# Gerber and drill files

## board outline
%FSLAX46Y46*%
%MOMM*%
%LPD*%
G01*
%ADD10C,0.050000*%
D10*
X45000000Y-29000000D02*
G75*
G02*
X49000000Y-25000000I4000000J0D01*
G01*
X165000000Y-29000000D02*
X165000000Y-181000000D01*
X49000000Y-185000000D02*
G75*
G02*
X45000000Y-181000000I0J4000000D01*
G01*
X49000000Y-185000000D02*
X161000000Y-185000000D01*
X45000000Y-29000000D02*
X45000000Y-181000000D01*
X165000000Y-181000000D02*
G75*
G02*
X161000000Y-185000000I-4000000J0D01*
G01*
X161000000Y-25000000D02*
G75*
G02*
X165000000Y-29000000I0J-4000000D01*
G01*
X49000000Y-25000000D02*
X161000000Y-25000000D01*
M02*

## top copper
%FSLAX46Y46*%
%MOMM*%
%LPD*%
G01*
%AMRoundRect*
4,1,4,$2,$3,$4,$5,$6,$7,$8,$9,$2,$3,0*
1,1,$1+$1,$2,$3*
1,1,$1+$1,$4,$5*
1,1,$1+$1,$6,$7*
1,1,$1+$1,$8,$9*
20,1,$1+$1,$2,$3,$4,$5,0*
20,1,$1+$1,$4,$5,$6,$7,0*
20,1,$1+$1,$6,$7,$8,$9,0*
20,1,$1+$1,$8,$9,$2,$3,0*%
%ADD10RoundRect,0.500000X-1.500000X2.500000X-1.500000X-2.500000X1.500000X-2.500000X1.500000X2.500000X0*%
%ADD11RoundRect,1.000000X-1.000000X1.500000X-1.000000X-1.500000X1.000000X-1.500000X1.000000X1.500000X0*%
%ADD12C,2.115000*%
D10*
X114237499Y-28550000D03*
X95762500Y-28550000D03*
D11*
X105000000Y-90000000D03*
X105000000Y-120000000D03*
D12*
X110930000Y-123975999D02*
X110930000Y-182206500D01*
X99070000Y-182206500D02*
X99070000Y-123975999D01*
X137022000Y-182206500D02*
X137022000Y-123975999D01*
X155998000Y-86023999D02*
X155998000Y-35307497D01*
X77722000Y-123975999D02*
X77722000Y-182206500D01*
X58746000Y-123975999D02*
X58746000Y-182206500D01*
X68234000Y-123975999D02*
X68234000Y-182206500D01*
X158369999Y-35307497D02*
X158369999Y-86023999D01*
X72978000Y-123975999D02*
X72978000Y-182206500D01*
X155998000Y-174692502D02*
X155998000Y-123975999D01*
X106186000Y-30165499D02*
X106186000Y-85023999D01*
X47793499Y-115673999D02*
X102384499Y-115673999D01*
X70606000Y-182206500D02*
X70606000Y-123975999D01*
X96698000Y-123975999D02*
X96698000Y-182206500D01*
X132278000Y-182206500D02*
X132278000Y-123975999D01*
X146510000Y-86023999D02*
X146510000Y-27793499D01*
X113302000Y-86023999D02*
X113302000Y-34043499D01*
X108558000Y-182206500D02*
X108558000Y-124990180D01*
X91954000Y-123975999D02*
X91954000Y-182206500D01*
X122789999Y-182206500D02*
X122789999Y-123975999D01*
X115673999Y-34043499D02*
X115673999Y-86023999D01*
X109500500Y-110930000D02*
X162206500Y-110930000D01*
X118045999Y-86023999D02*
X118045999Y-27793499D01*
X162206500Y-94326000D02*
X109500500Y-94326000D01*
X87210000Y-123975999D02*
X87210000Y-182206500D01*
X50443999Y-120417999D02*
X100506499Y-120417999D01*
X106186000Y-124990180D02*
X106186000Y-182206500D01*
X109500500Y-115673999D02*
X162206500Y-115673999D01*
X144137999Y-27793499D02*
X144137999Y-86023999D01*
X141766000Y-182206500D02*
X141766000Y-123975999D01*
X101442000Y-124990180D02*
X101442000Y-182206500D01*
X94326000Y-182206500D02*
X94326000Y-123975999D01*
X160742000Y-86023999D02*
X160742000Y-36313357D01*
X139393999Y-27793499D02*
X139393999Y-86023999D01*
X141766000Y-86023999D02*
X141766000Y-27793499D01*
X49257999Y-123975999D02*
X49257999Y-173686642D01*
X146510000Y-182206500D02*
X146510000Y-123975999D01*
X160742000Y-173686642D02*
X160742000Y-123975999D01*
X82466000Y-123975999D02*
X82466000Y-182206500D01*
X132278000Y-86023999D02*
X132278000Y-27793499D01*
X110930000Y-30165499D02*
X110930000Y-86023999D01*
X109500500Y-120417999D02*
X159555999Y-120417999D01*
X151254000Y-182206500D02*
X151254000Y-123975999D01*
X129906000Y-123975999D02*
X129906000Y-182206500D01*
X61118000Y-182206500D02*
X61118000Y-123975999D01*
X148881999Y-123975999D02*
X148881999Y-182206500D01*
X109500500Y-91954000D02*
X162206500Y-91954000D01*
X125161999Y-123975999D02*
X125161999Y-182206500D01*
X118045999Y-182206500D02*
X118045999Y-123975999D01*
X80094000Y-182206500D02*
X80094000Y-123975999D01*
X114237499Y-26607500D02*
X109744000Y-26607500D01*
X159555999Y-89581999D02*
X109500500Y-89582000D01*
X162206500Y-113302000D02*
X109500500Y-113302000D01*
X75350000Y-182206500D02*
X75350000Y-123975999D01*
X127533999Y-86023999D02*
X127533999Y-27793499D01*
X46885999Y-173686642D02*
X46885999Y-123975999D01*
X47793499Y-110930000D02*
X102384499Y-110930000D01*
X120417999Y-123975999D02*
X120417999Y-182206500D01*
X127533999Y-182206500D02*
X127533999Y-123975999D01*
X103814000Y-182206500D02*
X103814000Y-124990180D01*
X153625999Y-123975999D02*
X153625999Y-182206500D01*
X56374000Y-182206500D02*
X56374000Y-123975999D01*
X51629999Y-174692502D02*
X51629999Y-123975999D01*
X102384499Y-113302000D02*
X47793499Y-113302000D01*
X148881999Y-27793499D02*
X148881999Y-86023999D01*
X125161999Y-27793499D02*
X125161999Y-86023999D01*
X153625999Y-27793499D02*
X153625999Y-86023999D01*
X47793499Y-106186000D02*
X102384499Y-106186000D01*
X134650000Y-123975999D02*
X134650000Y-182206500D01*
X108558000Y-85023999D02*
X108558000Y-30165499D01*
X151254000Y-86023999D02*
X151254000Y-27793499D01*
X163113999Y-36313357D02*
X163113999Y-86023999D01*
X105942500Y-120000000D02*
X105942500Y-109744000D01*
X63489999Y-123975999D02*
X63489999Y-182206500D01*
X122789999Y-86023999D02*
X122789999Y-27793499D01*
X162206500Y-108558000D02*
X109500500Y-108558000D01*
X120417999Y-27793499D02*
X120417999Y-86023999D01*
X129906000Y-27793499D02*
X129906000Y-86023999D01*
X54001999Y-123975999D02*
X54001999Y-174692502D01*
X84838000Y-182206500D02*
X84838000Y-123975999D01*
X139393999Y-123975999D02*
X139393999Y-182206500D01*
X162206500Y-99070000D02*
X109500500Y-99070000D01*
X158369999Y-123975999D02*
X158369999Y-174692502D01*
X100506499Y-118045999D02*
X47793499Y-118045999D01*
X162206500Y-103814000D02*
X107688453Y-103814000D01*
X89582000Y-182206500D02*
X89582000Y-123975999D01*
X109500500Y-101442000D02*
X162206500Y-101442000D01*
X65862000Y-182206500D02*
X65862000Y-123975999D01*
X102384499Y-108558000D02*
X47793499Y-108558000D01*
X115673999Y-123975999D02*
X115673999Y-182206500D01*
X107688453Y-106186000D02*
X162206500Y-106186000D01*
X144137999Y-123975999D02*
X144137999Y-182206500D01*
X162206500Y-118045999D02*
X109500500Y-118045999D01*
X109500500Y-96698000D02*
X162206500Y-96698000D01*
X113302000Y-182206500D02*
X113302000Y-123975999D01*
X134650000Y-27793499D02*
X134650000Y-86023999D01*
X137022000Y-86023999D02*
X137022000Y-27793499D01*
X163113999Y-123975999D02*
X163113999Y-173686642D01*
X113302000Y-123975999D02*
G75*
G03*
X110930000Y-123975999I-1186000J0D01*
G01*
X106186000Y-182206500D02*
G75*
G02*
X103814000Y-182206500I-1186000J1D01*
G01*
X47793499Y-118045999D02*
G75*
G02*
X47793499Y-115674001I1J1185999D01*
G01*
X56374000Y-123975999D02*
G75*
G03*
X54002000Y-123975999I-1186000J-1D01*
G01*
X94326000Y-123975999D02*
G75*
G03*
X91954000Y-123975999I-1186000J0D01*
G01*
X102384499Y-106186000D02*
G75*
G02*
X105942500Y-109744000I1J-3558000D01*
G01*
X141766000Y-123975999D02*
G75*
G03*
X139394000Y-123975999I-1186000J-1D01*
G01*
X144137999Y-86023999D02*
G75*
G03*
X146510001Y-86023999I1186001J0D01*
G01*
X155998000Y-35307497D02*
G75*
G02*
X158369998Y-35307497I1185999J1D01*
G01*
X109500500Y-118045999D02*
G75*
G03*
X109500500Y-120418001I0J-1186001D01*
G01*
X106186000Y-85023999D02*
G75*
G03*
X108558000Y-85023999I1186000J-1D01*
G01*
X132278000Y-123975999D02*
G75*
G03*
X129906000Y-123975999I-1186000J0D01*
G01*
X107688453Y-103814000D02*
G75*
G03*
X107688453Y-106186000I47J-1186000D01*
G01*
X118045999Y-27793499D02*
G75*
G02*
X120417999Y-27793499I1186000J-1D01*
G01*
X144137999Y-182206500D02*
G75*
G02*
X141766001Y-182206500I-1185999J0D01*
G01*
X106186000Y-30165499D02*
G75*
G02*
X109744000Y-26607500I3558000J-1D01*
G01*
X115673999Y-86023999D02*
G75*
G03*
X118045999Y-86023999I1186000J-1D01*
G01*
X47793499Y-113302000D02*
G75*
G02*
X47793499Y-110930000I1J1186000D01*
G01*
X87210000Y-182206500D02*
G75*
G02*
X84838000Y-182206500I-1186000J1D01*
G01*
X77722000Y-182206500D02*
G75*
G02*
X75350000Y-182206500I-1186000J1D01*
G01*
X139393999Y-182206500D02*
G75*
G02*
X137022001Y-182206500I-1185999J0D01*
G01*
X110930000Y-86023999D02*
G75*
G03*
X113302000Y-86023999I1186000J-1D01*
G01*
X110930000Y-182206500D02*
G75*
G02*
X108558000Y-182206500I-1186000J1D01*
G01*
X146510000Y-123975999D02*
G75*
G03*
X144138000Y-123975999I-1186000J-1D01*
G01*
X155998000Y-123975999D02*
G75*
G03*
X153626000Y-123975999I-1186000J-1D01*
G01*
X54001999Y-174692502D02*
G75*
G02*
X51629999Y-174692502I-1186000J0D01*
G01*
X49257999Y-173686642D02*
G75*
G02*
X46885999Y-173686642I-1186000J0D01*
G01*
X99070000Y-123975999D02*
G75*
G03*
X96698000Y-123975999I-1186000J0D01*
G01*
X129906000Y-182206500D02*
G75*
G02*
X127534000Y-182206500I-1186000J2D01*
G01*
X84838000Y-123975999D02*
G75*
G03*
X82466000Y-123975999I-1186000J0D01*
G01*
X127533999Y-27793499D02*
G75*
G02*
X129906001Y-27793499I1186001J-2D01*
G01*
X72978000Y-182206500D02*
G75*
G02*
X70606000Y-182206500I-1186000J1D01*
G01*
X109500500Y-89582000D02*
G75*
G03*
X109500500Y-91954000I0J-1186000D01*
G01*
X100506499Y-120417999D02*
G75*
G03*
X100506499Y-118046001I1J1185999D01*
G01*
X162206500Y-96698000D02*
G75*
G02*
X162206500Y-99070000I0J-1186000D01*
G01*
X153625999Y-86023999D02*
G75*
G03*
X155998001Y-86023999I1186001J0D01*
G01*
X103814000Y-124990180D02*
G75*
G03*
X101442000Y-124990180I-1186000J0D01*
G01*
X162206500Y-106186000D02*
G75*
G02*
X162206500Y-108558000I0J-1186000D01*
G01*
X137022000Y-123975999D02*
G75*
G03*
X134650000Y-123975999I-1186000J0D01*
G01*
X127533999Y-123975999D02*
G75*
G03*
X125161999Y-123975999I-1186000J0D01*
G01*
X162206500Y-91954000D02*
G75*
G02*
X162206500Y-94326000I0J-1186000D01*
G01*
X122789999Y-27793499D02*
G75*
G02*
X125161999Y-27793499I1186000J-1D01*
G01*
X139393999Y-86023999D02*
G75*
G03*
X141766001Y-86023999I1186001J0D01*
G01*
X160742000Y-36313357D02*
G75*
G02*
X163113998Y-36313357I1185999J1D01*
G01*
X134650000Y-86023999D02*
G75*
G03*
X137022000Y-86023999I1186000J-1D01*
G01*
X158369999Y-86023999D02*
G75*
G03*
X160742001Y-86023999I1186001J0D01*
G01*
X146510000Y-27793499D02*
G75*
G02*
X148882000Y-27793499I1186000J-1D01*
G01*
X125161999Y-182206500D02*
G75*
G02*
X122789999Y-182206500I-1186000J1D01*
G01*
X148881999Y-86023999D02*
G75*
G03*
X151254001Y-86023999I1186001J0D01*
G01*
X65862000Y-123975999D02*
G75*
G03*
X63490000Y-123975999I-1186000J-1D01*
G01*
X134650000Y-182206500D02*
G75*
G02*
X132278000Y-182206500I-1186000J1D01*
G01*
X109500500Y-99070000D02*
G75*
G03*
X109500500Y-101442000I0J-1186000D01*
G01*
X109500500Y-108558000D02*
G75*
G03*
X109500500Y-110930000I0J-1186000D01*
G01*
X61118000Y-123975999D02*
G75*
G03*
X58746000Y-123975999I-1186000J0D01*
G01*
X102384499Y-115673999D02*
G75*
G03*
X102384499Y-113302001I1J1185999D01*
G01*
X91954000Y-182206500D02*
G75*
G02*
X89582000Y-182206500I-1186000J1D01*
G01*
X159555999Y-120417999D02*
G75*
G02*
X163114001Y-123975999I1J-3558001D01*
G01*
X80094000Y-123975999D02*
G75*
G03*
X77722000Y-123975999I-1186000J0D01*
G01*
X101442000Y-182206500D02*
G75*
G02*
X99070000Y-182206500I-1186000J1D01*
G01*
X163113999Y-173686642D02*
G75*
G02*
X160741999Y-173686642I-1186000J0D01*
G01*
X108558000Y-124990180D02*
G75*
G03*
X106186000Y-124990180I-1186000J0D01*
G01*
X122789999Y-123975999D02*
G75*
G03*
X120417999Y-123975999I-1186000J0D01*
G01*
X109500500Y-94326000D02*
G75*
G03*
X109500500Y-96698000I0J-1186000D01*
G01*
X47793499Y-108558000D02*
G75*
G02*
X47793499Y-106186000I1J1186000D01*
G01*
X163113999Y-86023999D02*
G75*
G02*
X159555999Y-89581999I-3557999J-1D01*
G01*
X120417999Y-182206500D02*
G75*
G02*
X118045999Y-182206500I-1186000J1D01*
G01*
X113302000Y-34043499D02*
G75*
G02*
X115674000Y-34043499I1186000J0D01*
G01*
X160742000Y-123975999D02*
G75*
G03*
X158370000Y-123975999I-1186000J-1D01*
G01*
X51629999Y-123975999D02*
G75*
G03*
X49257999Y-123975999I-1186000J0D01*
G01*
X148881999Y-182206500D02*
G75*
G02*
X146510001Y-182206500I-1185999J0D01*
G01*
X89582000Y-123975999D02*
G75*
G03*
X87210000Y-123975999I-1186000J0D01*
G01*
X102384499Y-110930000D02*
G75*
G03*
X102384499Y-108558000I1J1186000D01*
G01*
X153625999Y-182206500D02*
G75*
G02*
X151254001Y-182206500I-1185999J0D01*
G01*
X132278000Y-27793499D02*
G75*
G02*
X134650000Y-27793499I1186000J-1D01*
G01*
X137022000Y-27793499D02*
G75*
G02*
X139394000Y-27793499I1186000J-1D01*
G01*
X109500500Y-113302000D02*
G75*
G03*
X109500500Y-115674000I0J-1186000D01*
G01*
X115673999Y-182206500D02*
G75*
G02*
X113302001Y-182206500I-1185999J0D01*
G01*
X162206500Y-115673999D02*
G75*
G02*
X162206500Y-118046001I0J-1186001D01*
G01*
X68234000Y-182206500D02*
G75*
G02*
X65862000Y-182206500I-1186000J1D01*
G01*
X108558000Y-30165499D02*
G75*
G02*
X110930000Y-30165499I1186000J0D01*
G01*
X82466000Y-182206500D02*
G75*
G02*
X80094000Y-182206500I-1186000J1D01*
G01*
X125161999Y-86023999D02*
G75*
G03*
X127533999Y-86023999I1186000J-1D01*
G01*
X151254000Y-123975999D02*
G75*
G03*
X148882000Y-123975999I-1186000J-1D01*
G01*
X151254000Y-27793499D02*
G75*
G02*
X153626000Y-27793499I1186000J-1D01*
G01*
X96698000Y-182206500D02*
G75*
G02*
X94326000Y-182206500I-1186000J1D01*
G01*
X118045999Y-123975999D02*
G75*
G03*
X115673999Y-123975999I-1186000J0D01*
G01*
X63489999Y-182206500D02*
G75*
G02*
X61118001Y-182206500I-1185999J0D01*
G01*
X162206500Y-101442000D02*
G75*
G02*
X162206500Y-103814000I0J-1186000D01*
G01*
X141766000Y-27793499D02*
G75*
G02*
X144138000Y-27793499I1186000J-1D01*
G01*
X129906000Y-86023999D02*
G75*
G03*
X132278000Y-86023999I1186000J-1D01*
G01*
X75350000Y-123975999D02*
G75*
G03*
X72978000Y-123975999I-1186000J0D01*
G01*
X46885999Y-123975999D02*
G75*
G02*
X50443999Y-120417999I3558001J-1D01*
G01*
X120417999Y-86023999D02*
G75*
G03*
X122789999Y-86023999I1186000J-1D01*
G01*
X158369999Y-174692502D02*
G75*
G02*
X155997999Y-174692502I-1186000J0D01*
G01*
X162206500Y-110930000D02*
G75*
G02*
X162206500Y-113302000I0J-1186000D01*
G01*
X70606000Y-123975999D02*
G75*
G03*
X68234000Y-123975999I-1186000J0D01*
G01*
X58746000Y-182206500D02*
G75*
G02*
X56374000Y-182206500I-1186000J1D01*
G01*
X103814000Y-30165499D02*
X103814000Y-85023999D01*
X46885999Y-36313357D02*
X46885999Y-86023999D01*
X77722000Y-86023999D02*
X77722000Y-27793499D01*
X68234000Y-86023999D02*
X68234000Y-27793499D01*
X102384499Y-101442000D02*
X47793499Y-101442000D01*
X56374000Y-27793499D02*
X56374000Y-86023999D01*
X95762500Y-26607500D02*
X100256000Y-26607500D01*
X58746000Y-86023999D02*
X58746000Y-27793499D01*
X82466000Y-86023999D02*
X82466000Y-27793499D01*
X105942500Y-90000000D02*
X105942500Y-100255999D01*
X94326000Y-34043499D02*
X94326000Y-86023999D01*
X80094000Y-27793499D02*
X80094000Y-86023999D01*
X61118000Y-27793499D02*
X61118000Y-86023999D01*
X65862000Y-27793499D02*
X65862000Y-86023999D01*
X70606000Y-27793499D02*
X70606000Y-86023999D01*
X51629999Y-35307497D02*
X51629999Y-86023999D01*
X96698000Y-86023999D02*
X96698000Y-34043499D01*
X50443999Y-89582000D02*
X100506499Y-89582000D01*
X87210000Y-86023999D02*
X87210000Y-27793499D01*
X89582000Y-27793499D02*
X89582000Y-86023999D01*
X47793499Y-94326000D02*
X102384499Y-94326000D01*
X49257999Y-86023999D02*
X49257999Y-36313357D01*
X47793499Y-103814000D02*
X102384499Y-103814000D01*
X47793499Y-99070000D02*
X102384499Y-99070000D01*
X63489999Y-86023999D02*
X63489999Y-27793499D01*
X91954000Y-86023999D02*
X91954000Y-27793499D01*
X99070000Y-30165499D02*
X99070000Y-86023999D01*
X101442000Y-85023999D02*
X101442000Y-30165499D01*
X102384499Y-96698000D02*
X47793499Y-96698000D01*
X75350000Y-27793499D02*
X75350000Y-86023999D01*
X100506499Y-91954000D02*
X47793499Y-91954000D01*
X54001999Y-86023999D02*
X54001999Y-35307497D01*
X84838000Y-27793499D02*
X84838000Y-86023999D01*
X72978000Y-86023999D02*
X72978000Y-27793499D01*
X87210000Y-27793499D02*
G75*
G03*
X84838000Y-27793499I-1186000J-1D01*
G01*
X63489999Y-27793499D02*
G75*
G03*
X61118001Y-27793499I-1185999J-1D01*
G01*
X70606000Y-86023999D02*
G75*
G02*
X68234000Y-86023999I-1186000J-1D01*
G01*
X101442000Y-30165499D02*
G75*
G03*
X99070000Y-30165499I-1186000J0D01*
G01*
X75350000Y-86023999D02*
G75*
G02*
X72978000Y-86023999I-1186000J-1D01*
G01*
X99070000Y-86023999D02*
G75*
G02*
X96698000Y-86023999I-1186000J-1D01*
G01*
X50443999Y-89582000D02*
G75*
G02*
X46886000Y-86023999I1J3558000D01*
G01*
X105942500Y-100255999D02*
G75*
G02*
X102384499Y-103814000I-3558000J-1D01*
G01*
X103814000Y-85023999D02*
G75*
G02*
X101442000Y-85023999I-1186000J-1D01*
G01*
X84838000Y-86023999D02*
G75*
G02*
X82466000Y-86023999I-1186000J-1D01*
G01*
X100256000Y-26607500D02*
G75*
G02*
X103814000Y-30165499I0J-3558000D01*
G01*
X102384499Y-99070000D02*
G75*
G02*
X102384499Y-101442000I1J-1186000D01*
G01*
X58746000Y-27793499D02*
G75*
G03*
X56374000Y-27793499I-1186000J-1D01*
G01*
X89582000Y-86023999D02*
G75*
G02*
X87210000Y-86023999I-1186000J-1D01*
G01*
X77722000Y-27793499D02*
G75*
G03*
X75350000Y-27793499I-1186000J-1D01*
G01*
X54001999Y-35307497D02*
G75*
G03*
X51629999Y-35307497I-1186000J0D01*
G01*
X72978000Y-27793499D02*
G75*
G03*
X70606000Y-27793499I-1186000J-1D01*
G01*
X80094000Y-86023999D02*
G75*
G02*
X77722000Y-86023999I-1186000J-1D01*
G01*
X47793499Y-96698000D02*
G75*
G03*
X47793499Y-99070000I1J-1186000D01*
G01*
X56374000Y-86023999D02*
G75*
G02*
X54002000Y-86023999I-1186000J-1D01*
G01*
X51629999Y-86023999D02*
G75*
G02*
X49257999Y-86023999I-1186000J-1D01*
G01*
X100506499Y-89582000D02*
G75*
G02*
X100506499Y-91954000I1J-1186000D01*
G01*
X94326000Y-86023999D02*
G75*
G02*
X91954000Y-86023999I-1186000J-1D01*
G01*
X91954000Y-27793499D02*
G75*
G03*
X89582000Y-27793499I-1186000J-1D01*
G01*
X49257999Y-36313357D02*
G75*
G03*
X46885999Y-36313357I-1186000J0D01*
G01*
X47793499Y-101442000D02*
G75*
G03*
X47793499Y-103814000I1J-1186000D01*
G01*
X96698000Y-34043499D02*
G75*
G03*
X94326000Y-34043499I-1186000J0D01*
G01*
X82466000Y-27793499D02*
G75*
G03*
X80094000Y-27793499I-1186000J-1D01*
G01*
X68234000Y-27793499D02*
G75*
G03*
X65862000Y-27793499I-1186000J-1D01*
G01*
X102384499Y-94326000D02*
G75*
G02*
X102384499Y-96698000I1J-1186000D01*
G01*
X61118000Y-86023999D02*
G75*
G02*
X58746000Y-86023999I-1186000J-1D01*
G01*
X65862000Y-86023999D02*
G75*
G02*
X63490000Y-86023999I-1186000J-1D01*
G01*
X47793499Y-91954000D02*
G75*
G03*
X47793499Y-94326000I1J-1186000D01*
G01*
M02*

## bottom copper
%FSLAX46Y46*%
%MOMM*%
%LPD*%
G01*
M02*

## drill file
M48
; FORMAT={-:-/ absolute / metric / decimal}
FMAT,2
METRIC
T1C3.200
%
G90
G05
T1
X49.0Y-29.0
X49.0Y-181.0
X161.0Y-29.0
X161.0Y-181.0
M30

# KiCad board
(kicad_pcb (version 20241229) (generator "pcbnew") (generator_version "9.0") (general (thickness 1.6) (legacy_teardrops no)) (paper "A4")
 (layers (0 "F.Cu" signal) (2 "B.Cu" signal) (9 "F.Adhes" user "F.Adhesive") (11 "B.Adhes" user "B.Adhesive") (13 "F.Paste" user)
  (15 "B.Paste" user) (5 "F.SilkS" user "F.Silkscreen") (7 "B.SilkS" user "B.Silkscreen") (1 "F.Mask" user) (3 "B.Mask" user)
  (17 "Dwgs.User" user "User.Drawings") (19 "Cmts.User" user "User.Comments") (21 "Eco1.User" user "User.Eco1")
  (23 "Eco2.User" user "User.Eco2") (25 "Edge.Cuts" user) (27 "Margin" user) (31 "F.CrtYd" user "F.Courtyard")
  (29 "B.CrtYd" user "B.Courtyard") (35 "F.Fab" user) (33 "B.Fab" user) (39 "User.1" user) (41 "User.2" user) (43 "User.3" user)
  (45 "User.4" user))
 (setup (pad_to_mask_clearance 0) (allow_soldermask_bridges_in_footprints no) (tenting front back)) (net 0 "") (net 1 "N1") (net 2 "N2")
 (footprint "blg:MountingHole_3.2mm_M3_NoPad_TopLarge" (layer "F.Cu") (at 161 29)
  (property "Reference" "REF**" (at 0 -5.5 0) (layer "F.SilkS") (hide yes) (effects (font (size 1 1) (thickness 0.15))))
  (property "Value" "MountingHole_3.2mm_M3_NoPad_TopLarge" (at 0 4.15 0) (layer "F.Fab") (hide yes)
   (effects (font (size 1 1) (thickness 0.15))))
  (pad "" np_thru_hole circle (at 0 0) (size 7.6 7.6) (drill 3.2) (layers) (zone_connect 2)))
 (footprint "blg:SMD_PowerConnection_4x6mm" (layer "F.Cu") (at 114.237499 28.55 -90)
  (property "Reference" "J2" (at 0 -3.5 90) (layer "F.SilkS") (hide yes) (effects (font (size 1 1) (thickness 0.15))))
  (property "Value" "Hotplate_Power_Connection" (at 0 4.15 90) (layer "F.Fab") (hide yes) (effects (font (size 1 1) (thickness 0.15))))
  (pad "1" smd roundrect (at 0 0 270) (size 6 4) (layers "F.Cu" "F.Mask" "F.Paste") (roundrect_rratio 0.125) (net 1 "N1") (zone_connect 2)))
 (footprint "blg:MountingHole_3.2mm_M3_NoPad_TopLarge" (layer "F.Cu") (at 49 181)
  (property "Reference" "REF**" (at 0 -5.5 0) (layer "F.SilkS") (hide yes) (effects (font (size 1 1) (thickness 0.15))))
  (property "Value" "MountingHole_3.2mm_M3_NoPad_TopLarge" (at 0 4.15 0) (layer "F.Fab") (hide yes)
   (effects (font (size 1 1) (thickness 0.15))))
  (pad "" np_thru_hole circle (at 0 0) (size 7.6 7.6) (drill 3.2) (layers) (zone_connect 2)))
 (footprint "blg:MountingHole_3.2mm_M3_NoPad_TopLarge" (layer "F.Cu") (at 161 181)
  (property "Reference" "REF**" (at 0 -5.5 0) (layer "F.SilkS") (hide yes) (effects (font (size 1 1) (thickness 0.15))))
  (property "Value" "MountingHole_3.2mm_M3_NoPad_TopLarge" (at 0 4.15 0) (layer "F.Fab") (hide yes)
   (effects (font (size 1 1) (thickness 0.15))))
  (pad "" np_thru_hole circle (at 0 0) (size 7.6 7.6) (drill 3.2) (layers) (zone_connect 2)))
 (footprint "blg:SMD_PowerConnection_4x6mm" (layer "F.Cu") (at 95.7625 28.55 -90)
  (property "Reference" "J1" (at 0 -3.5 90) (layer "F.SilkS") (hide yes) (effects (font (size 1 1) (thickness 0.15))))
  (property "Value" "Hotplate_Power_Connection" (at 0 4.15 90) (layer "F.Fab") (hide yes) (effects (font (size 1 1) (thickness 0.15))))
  (pad "1" smd roundrect (at 0 0 270) (size 6 4) (layers "F.Cu" "F.Mask" "F.Paste") (roundrect_rratio 0.125) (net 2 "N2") (zone_connect 2)))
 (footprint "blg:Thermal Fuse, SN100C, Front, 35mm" (layer "F.Cu") (at 105 105 -90)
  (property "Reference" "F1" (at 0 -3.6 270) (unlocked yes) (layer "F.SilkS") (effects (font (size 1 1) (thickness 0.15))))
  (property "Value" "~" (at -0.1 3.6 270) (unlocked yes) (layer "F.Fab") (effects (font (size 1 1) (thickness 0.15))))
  (pad "1" smd roundrect (at -15 0 270) (size 5 4) (layers "F.Cu" "F.Mask") (roundrect_rratio 0.25) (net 2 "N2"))
  (pad "2" smd roundrect (at 15 0 270) (size 5 4) (layers "F.Cu" "F.Mask") (roundrect_rratio 0.25) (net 1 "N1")))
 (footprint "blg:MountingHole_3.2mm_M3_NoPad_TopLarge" (layer "F.Cu") (at 49 29)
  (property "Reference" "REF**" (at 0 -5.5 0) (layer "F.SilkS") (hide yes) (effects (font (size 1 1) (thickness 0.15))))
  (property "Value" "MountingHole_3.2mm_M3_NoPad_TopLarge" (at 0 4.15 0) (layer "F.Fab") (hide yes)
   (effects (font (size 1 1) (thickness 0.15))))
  (pad "" np_thru_hole circle (at 0 0) (size 7.6 7.6) (drill 3.2) (layers) (zone_connect 2)))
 (gr_arc (start 45 29) (mid 46.171573 26.171573) (end 49 25) (stroke (width 0.05) (type solid)) (layer "Edge.Cuts"))
 (gr_line (start 165 29) (end 165 181) (stroke (width 0.05) (type default)) (layer "Edge.Cuts"))
 (gr_arc (start 49 185) (mid 46.171573 183.828427) (end 45 181) (stroke (width 0.05) (type solid)) (layer "Edge.Cuts"))
 (gr_line (start 49 185) (end 161 185) (stroke (width 0.05) (type default)) (layer "Edge.Cuts"))
 (gr_line (start 45 29) (end 45 181) (stroke (width 0.05) (type default)) (layer "Edge.Cuts"))
 (gr_arc (start 165 181) (mid 163.828427 183.828427) (end 161 185) (stroke (width 0.05) (type solid)) (layer "Edge.Cuts"))
 (gr_arc (start 161 25) (mid 163.828427 26.171573) (end 165 29) (stroke (width 0.05) (type solid)) (layer "Edge.Cuts"))
 (gr_line (start 49 25) (end 161 25) (stroke (width 0.05) (type default)) (layer "Edge.Cuts"))
 (segment (start 110.93 123.975999) (end 110.93 182.2065) (width 2.115) (layer "F.Cu") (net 1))
 (segment (start 99.07 182.2065) (end 99.07 123.975999) (width 2.115) (layer "F.Cu") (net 1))
 (segment (start 137.022 182.2065) (end 137.022 123.975999) (width 2.115) (layer "F.Cu") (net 1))
 (segment (start 155.998 86.023999) (end 155.998 35.307497) (width 2.115) (layer "F.Cu") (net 1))
 (segment (start 77.722 123.975999) (end 77.722 182.2065) (width 2.115) (layer "F.Cu") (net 1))
 (segment (start 58.746 123.975999) (end 58.746 182.2065) (width 2.115) (layer "F.Cu") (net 1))
 (segment (start 68.234 123.975999) (end 68.234 182.2065) (width 2.115) (layer "F.Cu") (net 1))
 (segment (start 158.369999 35.307497) (end 158.369999 86.023999) (width 2.115) (layer "F.Cu") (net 1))
 (segment (start 72.978 123.975999) (end 72.978 182.2065) (width 2.115) (layer "F.Cu") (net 1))
 (segment (start 155.998 174.692502) (end 155.998 123.975999) (width 2.115) (layer "F.Cu") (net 1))
 (segment (start 106.186 30.165499) (end 106.186 85.023999) (width 2.115) (layer "F.Cu") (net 1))
 (segment (start 47.793499 115.673999) (end 102.384499 115.673999) (width 2.115) (layer "F.Cu") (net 1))
 (segment (start 70.606 182.2065) (end 70.606 123.975999) (width 2.115) (layer "F.Cu") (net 1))
 (segment (start 96.698 123.975999) (end 96.698 182.2065) (width 2.115) (layer "F.Cu") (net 1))
 (segment (start 132.278 182.2065) (end 132.278 123.975999) (width 2.115) (layer "F.Cu") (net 1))
 (segment (start 146.51 86.023999) (end 146.51 27.793499) (width 2.115) (layer "F.Cu") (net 1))
 (segment (start 113.302 86.023999) (end 113.302 34.043499) (width 2.115) (layer "F.Cu") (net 1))
 (segment (start 108.558 182.2065) (end 108.558 124.99018) (width 2.115) (layer "F.Cu") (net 1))
 (segment (start 91.954 123.975999) (end 91.954 182.2065) (width 2.115) (layer "F.Cu") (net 1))
 (segment (start 122.789999 182.2065) (end 122.789999 123.975999) (width 2.115) (layer "F.Cu") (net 1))
 (segment (start 115.673999 34.043499) (end 115.673999 86.023999) (width 2.115) (layer "F.Cu") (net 1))
 (segment (start 109.5005 110.93) (end 162.2065 110.93) (width 2.115) (layer "F.Cu") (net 1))
 (segment (start 118.045999 86.023999) (end 118.045999 27.793499) (width 2.115) (layer "F.Cu") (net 1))
 (segment (start 162.2065 94.326) (end 109.5005 94.326) (width 2.115) (layer "F.Cu") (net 1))
 (segment (start 87.21 123.975999) (end 87.21 182.2065) (width 2.115) (layer "F.Cu") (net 1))
 (segment (start 50.443999 120.417999) (end 100.506499 120.417999) (width 2.115) (layer "F.Cu") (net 1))
 (segment (start 106.186 124.99018) (end 106.186 182.2065) (width 2.115) (layer "F.Cu") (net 1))
 (segment (start 109.5005 115.673999) (end 162.2065 115.673999) (width 2.115) (layer "F.Cu") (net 1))
 (segment (start 144.137999 27.793499) (end 144.137999 86.023999) (width 2.115) (layer "F.Cu") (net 1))
 (segment (start 141.766 182.2065) (end 141.766 123.975999) (width 2.115) (layer "F.Cu") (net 1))
 (segment (start 101.442 124.99018) (end 101.442 182.2065) (width 2.115) (layer "F.Cu") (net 1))
 (segment (start 94.326 182.2065) (end 94.326 123.975999) (width 2.115) (layer "F.Cu") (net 1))
 (segment (start 160.742 86.023999) (end 160.742 36.313357) (width 2.115) (layer "F.Cu") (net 1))
 (segment (start 139.393999 27.793499) (end 139.393999 86.023999) (width 2.115) (layer "F.Cu") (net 1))
 (segment (start 141.766 86.023999) (end 141.766 27.793499) (width 2.115) (layer "F.Cu") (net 1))
 (segment (start 49.257999 123.975999) (end 49.257999 173.686642) (width 2.115) (layer "F.Cu") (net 1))
 (segment (start 146.51 182.2065) (end 146.51 123.975999) (width 2.115) (layer "F.Cu") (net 1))
 (segment (start 160.742 173.686642) (end 160.742 123.975999) (width 2.115) (layer "F.Cu") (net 1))
 (segment (start 82.466 123.975999) (end 82.466 182.2065) (width 2.115) (layer "F.Cu") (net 1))
 (segment (start 132.278 86.023999) (end 132.278 27.793499) (width 2.115) (layer "F.Cu") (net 1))
 (segment (start 110.93 30.165499) (end 110.93 86.023999) (width 2.115) (layer "F.Cu") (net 1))
 (segment (start 109.5005 120.417999) (end 159.555999 120.417999) (width 2.115) (layer "F.Cu") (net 1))
 (segment (start 151.254 182.2065) (end 151.254 123.975999) (width 2.115) (layer "F.Cu") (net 1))
 (segment (start 129.906 123.975999) (end 129.906 182.2065) (width 2.115) (layer "F.Cu") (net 1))
 (segment (start 61.118 182.2065) (end 61.118 123.975999) (width 2.115) (layer "F.Cu") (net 1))
 (segment (start 148.881999 123.975999) (end 148.881999 182.2065) (width 2.115) (layer "F.Cu") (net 1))
 (segment (start 109.5005 91.954) (end 162.2065 91.954) (width 2.115) (layer "F.Cu") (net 1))
 (segment (start 125.161999 123.975999) (end 125.161999 182.2065) (width 2.115) (layer "F.Cu") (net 1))
 (segment (start 118.045999 182.2065) (end 118.045999 123.975999) (width 2.115) (layer "F.Cu") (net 1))
 (segment (start 80.094 182.2065) (end 80.094 123.975999) (width 2.115) (layer "F.Cu") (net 1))
 (segment (start 114.237499 26.6075) (end 109.744 26.6075) (width 2.115) (layer "F.Cu") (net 1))
 (segment (start 159.555999 89.581999) (end 109.5005 89.582) (width 2.115) (layer "F.Cu") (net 1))
 (segment (start 162.2065 113.302) (end 109.5005 113.302) (width 2.115) (layer "F.Cu") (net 1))
 (segment (start 75.35 182.2065) (end 75.35 123.975999) (width 2.115) (layer "F.Cu") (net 1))
 (segment (start 127.533999 86.023999) (end 127.533999 27.793499) (width 2.115) (layer "F.Cu") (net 1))
 (segment (start 46.885999 173.686642) (end 46.885999 123.975999) (width 2.115) (layer "F.Cu") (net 1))
 (segment (start 47.793499 110.93) (end 102.384499 110.93) (width 2.115) (layer "F.Cu") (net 1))
 (segment (start 120.417999 123.975999) (end 120.417999 182.2065) (width 2.115) (layer "F.Cu") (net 1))
 (segment (start 127.533999 182.2065) (end 127.533999 123.975999) (width 2.115) (layer "F.Cu") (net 1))
 (segment (start 103.814 182.2065) (end 103.814 124.99018) (width 2.115) (layer "F.Cu") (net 1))
 (segment (start 153.625999 123.975999) (end 153.625999 182.2065) (width 2.115) (layer "F.Cu") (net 1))
 (segment (start 56.374 182.2065) (end 56.374 123.975999) (width 2.115) (layer "F.Cu") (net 1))
 (segment (start 51.629999 174.692502) (end 51.629999 123.975999) (width 2.115) (layer "F.Cu") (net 1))
 (segment (start 102.384499 113.302) (end 47.793499 113.302) (width 2.115) (layer "F.Cu") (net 1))
 (segment (start 148.881999 27.793499) (end 148.881999 86.023999) (width 2.115) (layer "F.Cu") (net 1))
 (segment (start 125.161999 27.793499) (end 125.161999 86.023999) (width 2.115) (layer "F.Cu") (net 1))
 (segment (start 153.625999 27.793499) (end 153.625999 86.023999) (width 2.115) (layer "F.Cu") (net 1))
 (segment (start 47.793499 106.186) (end 102.384499 106.186) (width 2.115) (layer "F.Cu") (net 1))
 (segment (start 134.65 123.975999) (end 134.65 182.2065) (width 2.115) (layer "F.Cu") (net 1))
 (segment (start 108.558 85.023999) (end 108.558 30.165499) (width 2.115) (layer "F.Cu") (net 1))
 (segment (start 151.254 86.023999) (end 151.254 27.793499) (width 2.115) (layer "F.Cu") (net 1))
 (segment (start 163.113999 36.313357) (end 163.113999 86.023999) (width 2.115) (layer "F.Cu") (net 1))
 (segment (start 105.9425 120) (end 105.9425 109.744) (width 2.115) (layer "F.Cu") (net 1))
 (segment (start 63.489999 123.975999) (end 63.489999 182.2065) (width 2.115) (layer "F.Cu") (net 1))
 (segment (start 122.789999 86.023999) (end 122.789999 27.793499) (width 2.115) (layer "F.Cu") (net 1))
 (segment (start 162.2065 108.558) (end 109.5005 108.558) (width 2.115) (layer "F.Cu") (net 1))
 (segment (start 120.417999 27.793499) (end 120.417999 86.023999) (width 2.115) (layer "F.Cu") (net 1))
 (segment (start 129.906 27.793499) (end 129.906 86.023999) (width 2.115) (layer "F.Cu") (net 1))
 (segment (start 54.001999 123.975999) (end 54.001999 174.692502) (width 2.115) (layer "F.Cu") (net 1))
 (segment (start 84.838 182.2065) (end 84.838 123.975999) (width 2.115) (layer "F.Cu") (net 1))
 (segment (start 139.393999 123.975999) (end 139.393999 182.2065) (width 2.115) (layer "F.Cu") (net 1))
 (segment (start 162.2065 99.07) (end 109.5005 99.07) (width 2.115) (layer "F.Cu") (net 1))
 (segment (start 158.369999 123.975999) (end 158.369999 174.692502) (width 2.115) (layer "F.Cu") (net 1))
 (segment (start 100.506499 118.045999) (end 47.793499 118.045999) (width 2.115) (layer "F.Cu") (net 1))
 (segment (start 162.2065 103.814) (end 107.688453 103.814) (width 2.115) (layer "F.Cu") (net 1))
 (segment (start 89.582 182.2065) (end 89.582 123.975999) (width 2.115) (layer "F.Cu") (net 1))
 (segment (start 109.5005 101.442) (end 162.2065 101.442) (width 2.115) (layer "F.Cu") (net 1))
 (segment (start 65.862 182.2065) (end 65.862 123.975999) (width 2.115) (layer "F.Cu") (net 1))
 (segment (start 102.384499 108.558) (end 47.793499 108.558) (width 2.115) (layer "F.Cu") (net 1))
 (segment (start 115.673999 123.975999) (end 115.673999 182.2065) (width 2.115) (layer "F.Cu") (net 1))
 (segment (start 107.688453 106.186) (end 162.2065 106.186) (width 2.115) (layer "F.Cu") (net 1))
 (segment (start 144.137999 123.975999) (end 144.137999 182.2065) (width 2.115) (layer "F.Cu") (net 1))
 (segment (start 162.2065 118.045999) (end 109.5005 118.045999) (width 2.115) (layer "F.Cu") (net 1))
 (segment (start 109.5005 96.698) (end 162.2065 96.698) (width 2.115) (layer "F.Cu") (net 1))
 (segment (start 113.302 182.2065) (end 113.302 123.975999) (width 2.115) (layer "F.Cu") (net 1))
 (segment (start 134.65 27.793499) (end 134.65 86.023999) (width 2.115) (layer "F.Cu") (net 1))
 (segment (start 137.022 86.023999) (end 137.022 27.793499) (width 2.115) (layer "F.Cu") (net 1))
 (segment (start 163.113999 123.975999) (end 163.113999 173.686642) (width 2.115) (layer "F.Cu") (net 1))
 (arc (start 113.302 123.975999) (mid 112.116 122.789999) (end 110.93 123.975999) (width 2.115) (layer "F.Cu") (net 1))
 (arc (start 106.186 182.2065) (mid 105 183.392499) (end 103.814 182.2065) (width 2.115) (layer "F.Cu") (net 1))
 (arc (start 47.793499 118.045999) (mid 46.607499 116.859999) (end 47.793499 115.673999) (width 2.115) (layer "F.Cu") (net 1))
 (arc (start 56.374 123.975999) (mid 55.188 122.789999) (end 54.001999 123.975999) (width 2.115) (layer "F.Cu") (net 1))
 (arc (start 94.326 123.975999) (mid 93.14 122.789999) (end 91.954 123.975999) (width 2.115) (layer "F.Cu") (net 1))
 (arc (start 102.384499 106.186) (mid 104.900385 107.228114) (end 105.9425 109.744) (width 2.115) (layer "F.Cu") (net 1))
 (arc (start 141.766 123.975999) (mid 140.579999 122.789999) (end 139.393999 123.975999) (width 2.115) (layer "F.Cu") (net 1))
 (arc (start 144.137999 86.023999) (mid 145.323999 87.21) (end 146.51 86.023999) (width 2.115) (layer "F.Cu") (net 1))
 (arc (start 155.998 35.307497) (mid 157.184 34.121497) (end 158.369999 35.307497) (width 2.115) (layer "F.Cu") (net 1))
 (arc (start 109.5005 118.045999) (mid 108.3145 119.231999) (end 109.5005 120.417999) (width 2.115) (layer "F.Cu") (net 1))
 (arc (start 106.186 85.023999) (mid 107.372 86.21) (end 108.558 85.023999) (width 2.115) (layer "F.Cu") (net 1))
 (arc (start 132.278 123.975999) (mid 131.091999 122.789999) (end 129.906 123.975999) (width 2.115) (layer "F.Cu") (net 1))
 (arc (start 107.688453 103.814) (mid 106.502453 105) (end 107.688453 106.186) (width 2.115) (layer "F.Cu") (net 1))
 (arc (start 118.045999 27.793499) (mid 119.231999 26.6075) (end 120.417999 27.793499) (width 2.115) (layer "F.Cu") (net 1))
 (arc (start 144.137999 182.2065) (mid 142.952 183.392499) (end 141.766 182.2065) (width 2.115) (layer "F.Cu") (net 1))
 (arc (start 106.186 30.165499) (mid 107.228114 27.649614) (end 109.744 26.6075) (width 2.115) (layer "F.Cu") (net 1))
 (arc (start 115.673999 86.023999) (mid 116.859999 87.21) (end 118.045999 86.023999) (width 2.115) (layer "F.Cu") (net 1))
 (arc (start 47.793499 113.302) (mid 46.607499 112.116) (end 47.793499 110.93) (width 2.115) (layer "F.Cu") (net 1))
 (arc (start 87.21 182.2065) (mid 86.023999 183.392499) (end 84.838 182.2065) (width 2.115) (layer "F.Cu") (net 1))
 (arc (start 77.722 182.2065) (mid 76.535999 183.392499) (end 75.35 182.2065) (width 2.115) (layer "F.Cu") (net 1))
 (arc (start 139.393999 182.2065) (mid 138.208 183.392499) (end 137.022 182.2065) (width 2.115) (layer "F.Cu") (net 1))
 (arc (start 110.93 86.023999) (mid 112.116 87.21) (end 113.302 86.023999) (width 2.115) (layer "F.Cu") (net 1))
 (arc (start 110.93 182.2065) (mid 109.744 183.392499) (end 108.558 182.2065) (width 2.115) (layer "F.Cu") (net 1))
 (arc (start 146.51 123.975999) (mid 145.323999 122.789999) (end 144.137999 123.975999) (width 2.115) (layer "F.Cu") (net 1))
 (arc (start 155.998 123.975999) (mid 154.812 122.789999) (end 153.625999 123.975999) (width 2.115) (layer "F.Cu") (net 1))
 (arc (start 54.001999 174.692502) (mid 52.815999 175.878502) (end 51.629999 174.692502) (width 2.115) (layer "F.Cu") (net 1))
 (arc (start 49.257999 173.686642) (mid 48.071999 174.872642) (end 46.885999 173.686642) (width 2.115) (layer "F.Cu") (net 1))
 (arc (start 99.07 123.975999) (mid 97.884 122.789999) (end 96.698 123.975999) (width 2.115) (layer "F.Cu") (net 1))
 (arc (start 129.906 182.2065) (mid 128.72 183.392499) (end 127.533999 182.2065) (width 2.115) (layer "F.Cu") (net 1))
 (arc (start 84.838 123.975999) (mid 83.651999 122.789999) (end 82.466 123.975999) (width 2.115) (layer "F.Cu") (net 1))
 (arc (start 127.533999 27.793499) (mid 128.72 26.6075) (end 129.906 27.793499) (width 2.115) (layer "F.Cu") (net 1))
 (arc (start 72.978 182.2065) (mid 71.792 183.392499) (end 70.606 182.2065) (width 2.115) (layer "F.Cu") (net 1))
 (arc (start 109.5005 89.582) (mid 108.3145 90.768) (end 109.5005 91.954) (width 2.115) (layer "F.Cu") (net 1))
 (arc (start 100.506499 120.417999) (mid 101.6925 119.231999) (end 100.506499 118.045999) (width 2.115) (layer "F.Cu") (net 1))
 (arc (start 162.2065 96.698) (mid 163.392499 97.884) (end 162.2065 99.07) (width 2.115) (layer "F.Cu") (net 1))
 (arc (start 153.625999 86.023999) (mid 154.812 87.21) (end 155.998 86.023999) (width 2.115) (layer "F.Cu") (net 1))
 (arc (start 103.814 124.99018) (mid 102.628 123.80418) (end 101.442 124.99018) (width 2.115) (layer "F.Cu") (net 1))
 (arc (start 162.2065 106.186) (mid 163.392499 107.372) (end 162.2065 108.558) (width 2.115) (layer "F.Cu") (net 1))
 (arc (start 137.022 123.975999) (mid 135.835999 122.789999) (end 134.65 123.975999) (width 2.115) (layer "F.Cu") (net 1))
 (arc (start 127.533999 123.975999) (mid 126.347999 122.789999) (end 125.161999 123.975999) (width 2.115) (layer "F.Cu") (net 1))
 (arc (start 162.2065 91.954) (mid 163.392499 93.14) (end 162.2065 94.326) (width 2.115) (layer "F.Cu") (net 1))
 (arc (start 122.789999 27.793499) (mid 123.975999 26.6075) (end 125.161999 27.793499) (width 2.115) (layer "F.Cu") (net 1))
 (arc (start 139.393999 86.023999) (mid 140.579999 87.21) (end 141.766 86.023999) (width 2.115) (layer "F.Cu") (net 1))
 (arc (start 160.742 36.313357) (mid 161.928 35.127357) (end 163.113999 36.313357) (width 2.115) (layer "F.Cu") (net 1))
 (arc (start 134.65 86.023999) (mid 135.835999 87.21) (end 137.022 86.023999) (width 2.115) (layer "F.Cu") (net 1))
 (arc (start 158.369999 86.023999) (mid 159.556 87.21) (end 160.742 86.023999) (width 2.115) (layer "F.Cu") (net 1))
 (arc (start 146.51 27.793499) (mid 147.696 26.6075) (end 148.881999 27.793499) (width 2.115) (layer "F.Cu") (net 1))
 (arc (start 125.161999 182.2065) (mid 123.975999 183.392499) (end 122.789999 182.2065) (width 2.115) (layer "F.Cu") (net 1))
 (arc (start 148.881999 86.023999) (mid 150.068 87.21) (end 151.254 86.023999) (width 2.115) (layer "F.Cu") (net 1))
 (arc (start 65.862 123.975999) (mid 64.676 122.789999) (end 63.489999 123.975999) (width 2.115) (layer "F.Cu") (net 1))
 (arc (start 134.65 182.2065) (mid 133.464 183.392499) (end 132.278 182.2065) (width 2.115) (layer "F.Cu") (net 1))
 (arc (start 109.5005 99.07) (mid 108.3145 100.256) (end 109.5005 101.442) (width 2.115) (layer "F.Cu") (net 1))
 (arc (start 109.5005 108.558) (mid 108.3145 109.744) (end 109.5005 110.93) (width 2.115) (layer "F.Cu") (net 1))
 (arc (start 61.118 123.975999) (mid 59.932 122.789999) (end 58.746 123.975999) (width 2.115) (layer "F.Cu") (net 1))
 (arc (start 102.384499 115.673999) (mid 103.5705 114.488) (end 102.384499 113.302) (width 2.115) (layer "F.Cu") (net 1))
 (arc (start 91.954 182.2065) (mid 90.768 183.392499) (end 89.582 182.2065) (width 2.115) (layer "F.Cu") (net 1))
 (arc (start 159.555999 120.417999) (mid 162.071885 121.460114) (end 163.113999 123.975999) (width 2.115) (layer "F.Cu") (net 1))
 (arc (start 80.094 123.975999) (mid 78.907999 122.789999) (end 77.722 123.975999) (width 2.115) (layer "F.Cu") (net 1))
 (arc (start 101.442 182.2065) (mid 100.256 183.392499) (end 99.07 182.2065) (width 2.115) (layer "F.Cu") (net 1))
 (arc (start 163.113999 173.686642) (mid 161.928 174.872642) (end 160.742 173.686642) (width 2.115) (layer "F.Cu") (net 1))
 (arc (start 108.558 124.99018) (mid 107.372 123.80418) (end 106.186 124.99018) (width 2.115) (layer "F.Cu") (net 1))
 (arc (start 122.789999 123.975999) (mid 121.603999 122.789999) (end 120.417999 123.975999) (width 2.115) (layer "F.Cu") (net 1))
 (arc (start 109.5005 94.326) (mid 108.3145 95.512) (end 109.5005 96.698) (width 2.115) (layer "F.Cu") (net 1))
 (arc (start 47.793499 108.558) (mid 46.607499 107.372) (end 47.793499 106.186) (width 2.115) (layer "F.Cu") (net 1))
 (arc (start 163.113999 86.023999) (mid 162.071885 88.539885) (end 159.555999 89.581999) (width 2.115) (layer "F.Cu") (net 1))
 (arc (start 120.417999 182.2065) (mid 119.231999 183.392499) (end 118.045999 182.2065) (width 2.115) (layer "F.Cu") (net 1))
 (arc (start 113.302 34.043499) (mid 114.488 32.857499) (end 115.673999 34.043499) (width 2.115) (layer "F.Cu") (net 1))
 (arc (start 160.742 123.975999) (mid 159.556 122.789999) (end 158.369999 123.975999) (width 2.115) (layer "F.Cu") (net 1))
 (arc (start 51.629999 123.975999) (mid 50.443999 122.789999) (end 49.257999 123.975999) (width 2.115) (layer "F.Cu") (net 1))
 (arc (start 148.881999 182.2065) (mid 147.696 183.392499) (end 146.51 182.2065) (width 2.115) (layer "F.Cu") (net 1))
 (arc (start 89.582 123.975999) (mid 88.396 122.789999) (end 87.21 123.975999) (width 2.115) (layer "F.Cu") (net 1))
 (arc (start 102.384499 110.93) (mid 103.5705 109.744) (end 102.384499 108.558) (width 2.115) (layer "F.Cu") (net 1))
 (arc (start 153.625999 182.2065) (mid 152.44 183.392499) (end 151.254 182.2065) (width 2.115) (layer "F.Cu") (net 1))
 (arc (start 132.278 27.793499) (mid 133.464 26.6075) (end 134.65 27.793499) (width 2.115) (layer "F.Cu") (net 1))
 (arc (start 137.022 27.793499) (mid 138.208 26.6075) (end 139.393999 27.793499) (width 2.115) (layer "F.Cu") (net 1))
 (arc (start 109.5005 113.302) (mid 108.3145 114.488) (end 109.5005 115.673999) (width 2.115) (layer "F.Cu") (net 1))
 (arc (start 115.673999 182.2065) (mid 114.488 183.392499) (end 113.302 182.2065) (width 2.115) (layer "F.Cu") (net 1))
 (arc (start 162.2065 115.673999) (mid 163.392499 116.859999) (end 162.2065 118.045999) (width 2.115) (layer "F.Cu") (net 1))
 (arc (start 68.234 182.2065) (mid 67.048 183.392499) (end 65.862 182.2065) (width 2.115) (layer "F.Cu") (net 1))
 (arc (start 108.558 30.165499) (mid 109.744 28.979499) (end 110.93 30.165499) (width 2.115) (layer "F.Cu") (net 1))
 (arc (start 82.466 182.2065) (mid 81.279999 183.392499) (end 80.094 182.2065) (width 2.115) (layer "F.Cu") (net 1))
 (arc (start 125.161999 86.023999) (mid 126.347999 87.21) (end 127.533999 86.023999) (width 2.115) (layer "F.Cu") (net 1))
 (arc (start 151.254 123.975999) (mid 150.068 122.789999) (end 148.881999 123.975999) (width 2.115) (layer "F.Cu") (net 1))
 (arc (start 151.254 27.793499) (mid 152.44 26.6075) (end 153.625999 27.793499) (width 2.115) (layer "F.Cu") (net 1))
 (arc (start 96.698 182.2065) (mid 95.512 183.392499) (end 94.326 182.2065) (width 2.115) (layer "F.Cu") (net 1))
 (arc (start 118.045999 123.975999) (mid 116.859999 122.789999) (end 115.673999 123.975999) (width 2.115) (layer "F.Cu") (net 1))
 (arc (start 63.489999 182.2065) (mid 62.303999 183.392499) (end 61.118 182.2065) (width 2.115) (layer "F.Cu") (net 1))
 (arc (start 162.2065 101.442) (mid 163.392499 102.628) (end 162.2065 103.814) (width 2.115) (layer "F.Cu") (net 1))
 (arc (start 141.766 27.793499) (mid 142.952 26.6075) (end 144.137999 27.793499) (width 2.115) (layer "F.Cu") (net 1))
 (arc (start 129.906 86.023999) (mid 131.091999 87.21) (end 132.278 86.023999) (width 2.115) (layer "F.Cu") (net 1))
 (arc (start 75.35 123.975999) (mid 74.163999 122.789999) (end 72.978 123.975999) (width 2.115) (layer "F.Cu") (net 1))
 (arc (start 46.885999 123.975999) (mid 47.928114 121.460114) (end 50.443999 120.417999) (width 2.115) (layer "F.Cu") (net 1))
 (arc (start 120.417999 86.023999) (mid 121.603999 87.21) (end 122.789999 86.023999) (width 2.115) (layer "F.Cu") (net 1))
 (arc (start 158.369999 174.692502) (mid 157.184 175.878502) (end 155.998 174.692502) (width 2.115) (layer "F.Cu") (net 1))
 (arc (start 162.2065 110.93) (mid 163.392499 112.116) (end 162.2065 113.302) (width 2.115) (layer "F.Cu") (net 1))
 (arc (start 70.606 123.975999) (mid 69.42 122.789999) (end 68.234 123.975999) (width 2.115) (layer "F.Cu") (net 1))
 (arc (start 58.746 182.2065) (mid 57.56 183.392499) (end 56.374 182.2065) (width 2.115) (layer "F.Cu") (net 1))
 (segment (start 103.814 30.165499) (end 103.814 85.023999) (width 2.115) (layer "F.Cu") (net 2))
 (segment (start 46.885999 36.313357) (end 46.885999 86.023999) (width 2.115) (layer "F.Cu") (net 2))
 (segment (start 77.722 86.023999) (end 77.722 27.793499) (width 2.115) (layer "F.Cu") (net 2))
 (segment (start 68.234 86.023999) (end 68.234 27.793499) (width 2.115) (layer "F.Cu") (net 2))
 (segment (start 102.384499 101.442) (end 47.793499 101.442) (width 2.115) (layer "F.Cu") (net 2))
 (segment (start 56.374 27.793499) (end 56.374 86.023999) (width 2.115) (layer "F.Cu") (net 2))
 (segment (start 95.7625 26.6075) (end 100.256 26.6075) (width 2.115) (layer "F.Cu") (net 2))
 (segment (start 58.746 86.023999) (end 58.746 27.793499) (width 2.115) (layer "F.Cu") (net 2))
 (segment (start 82.466 86.023999) (end 82.466 27.793499) (width 2.115) (layer "F.Cu") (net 2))
 (segment (start 105.9425 90) (end 105.9425 100.255999) (width 2.115) (layer "F.Cu") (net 2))
 (segment (start 94.326 34.043499) (end 94.326 86.023999) (width 2.115) (layer "F.Cu") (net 2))
 (segment (start 80.094 27.793499) (end 80.094 86.023999) (width 2.115) (layer "F.Cu") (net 2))
 (segment (start 61.118 27.793499) (end 61.118 86.023999) (width 2.115) (layer "F.Cu") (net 2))
 (segment (start 65.862 27.793499) (end 65.862 86.023999) (width 2.115) (layer "F.Cu") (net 2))
 (segment (start 70.606 27.793499) (end 70.606 86.023999) (width 2.115) (layer "F.Cu") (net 2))
 (segment (start 51.629999 35.307497) (end 51.629999 86.023999) (width 2.115) (layer "F.Cu") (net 2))
 (segment (start 96.698 86.023999) (end 96.698 34.043499) (width 2.115) (layer "F.Cu") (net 2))
 (segment (start 50.443999 89.582) (end 100.506499 89.582) (width 2.115) (layer "F.Cu") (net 2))
 (segment (start 87.21 86.023999) (end 87.21 27.793499) (width 2.115) (layer "F.Cu") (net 2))
 (segment (start 89.582 27.793499) (end 89.582 86.023999) (width 2.115) (layer "F.Cu") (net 2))
 (segment (start 47.793499 94.326) (end 102.384499 94.326) (width 2.115) (layer "F.Cu") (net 2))
 (segment (start 49.257999 86.023999) (end 49.257999 36.313357) (width 2.115) (layer "F.Cu") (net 2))
 (segment (start 47.793499 103.814) (end 102.384499 103.814) (width 2.115) (layer "F.Cu") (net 2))
 (segment (start 47.793499 99.07) (end 102.384499 99.07) (width 2.115) (layer "F.Cu") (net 2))
 (segment (start 63.489999 86.023999) (end 63.489999 27.793499) (width 2.115) (layer "F.Cu") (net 2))
 (segment (start 91.954 86.023999) (end 91.954 27.793499) (width 2.115) (layer "F.Cu") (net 2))
 (segment (start 99.07 30.165499) (end 99.07 86.023999) (width 2.115) (layer "F.Cu") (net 2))
 (segment (start 101.442 85.023999) (end 101.442 30.165499) (width 2.115) (layer "F.Cu") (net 2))
 (segment (start 102.384499 96.698) (end 47.793499 96.698) (width 2.115) (layer "F.Cu") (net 2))
 (segment (start 75.35 27.793499) (end 75.35 86.023999) (width 2.115) (layer "F.Cu") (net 2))
 (segment (start 100.506499 91.954) (end 47.793499 91.954) (width 2.115) (layer "F.Cu") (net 2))
 (segment (start 54.001999 86.023999) (end 54.001999 35.307497) (width 2.115) (layer "F.Cu") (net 2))
 (segment (start 84.838 27.793499) (end 84.838 86.023999) (width 2.115) (layer "F.Cu") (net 2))
 (segment (start 72.978 86.023999) (end 72.978 27.793499) (width 2.115) (layer "F.Cu") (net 2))
 (arc (start 87.21 27.793499) (mid 86.023999 26.6075) (end 84.838 27.793499) (width 2.115) (layer "F.Cu") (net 2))
 (arc (start 63.489999 27.793499) (mid 62.303999 26.6075) (end 61.118 27.793499) (width 2.115) (layer "F.Cu") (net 2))
 (arc (start 70.606 86.023999) (mid 69.42 87.21) (end 68.234 86.023999) (width 2.115) (layer "F.Cu") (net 2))
 (arc (start 101.442 30.165499) (mid 100.256 28.979499) (end 99.07 30.165499) (width 2.115) (layer "F.Cu") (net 2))
 (arc (start 75.35 86.023999) (mid 74.163999 87.21) (end 72.978 86.023999) (width 2.115) (layer "F.Cu") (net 2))
 (arc (start 99.07 86.023999) (mid 97.884 87.21) (end 96.698 86.023999) (width 2.115) (layer "F.Cu") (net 2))
 (arc (start 50.443999 89.582) (mid 47.928114 88.539885) (end 46.885999 86.023999) (width 2.115) (layer "F.Cu") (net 2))
 (arc (start 105.9425 100.255999) (mid 104.900385 102.771885) (end 102.384499 103.814) (width 2.115) (layer "F.Cu") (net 2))
 (arc (start 103.814 85.023999) (mid 102.628 86.21) (end 101.442 85.023999) (width 2.115) (layer "F.Cu") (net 2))
 (arc (start 84.838 86.023999) (mid 83.651999 87.21) (end 82.466 86.023999) (width 2.115) (layer "F.Cu") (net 2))
 (arc (start 100.256 26.6075) (mid 102.771885 27.649614) (end 103.814 30.165499) (width 2.115) (layer "F.Cu") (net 2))
 (arc (start 102.384499 99.07) (mid 103.5705 100.256) (end 102.384499 101.442) (width 2.115) (layer "F.Cu") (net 2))
 (arc (start 58.746 27.793499) (mid 57.56 26.6075) (end 56.374 27.793499) (width 2.115) (layer "F.Cu") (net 2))
 (arc (start 89.582 86.023999) (mid 88.396 87.21) (end 87.21 86.023999) (width 2.115) (layer "F.Cu") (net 2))
 (arc (start 77.722 27.793499) (mid 76.535999 26.6075) (end 75.35 27.793499) (width 2.115) (layer "F.Cu") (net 2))
 (arc (start 54.001999 35.307497) (mid 52.815999 34.121497) (end 51.629999 35.307497) (width 2.115) (layer "F.Cu") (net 2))
 (arc (start 72.978 27.793499) (mid 71.792 26.6075) (end 70.606 27.793499) (width 2.115) (layer "F.Cu") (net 2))
 (arc (start 80.094 86.023999) (mid 78.907999 87.21) (end 77.722 86.023999) (width 2.115) (layer "F.Cu") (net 2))
 (arc (start 47.793499 96.698) (mid 46.607499 97.884) (end 47.793499 99.07) (width 2.115) (layer "F.Cu") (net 2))
 (arc (start 56.374 86.023999) (mid 55.188 87.21) (end 54.001999 86.023999) (width 2.115) (layer "F.Cu") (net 2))
 (arc (start 51.629999 86.023999) (mid 50.443999 87.21) (end 49.257999 86.023999) (width 2.115) (layer "F.Cu") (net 2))
 (arc (start 100.506499 89.582) (mid 101.6925 90.768) (end 100.506499 91.954) (width 2.115) (layer "F.Cu") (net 2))
 (arc (start 94.326 86.023999) (mid 93.14 87.21) (end 91.954 86.023999) (width 2.115) (layer "F.Cu") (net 2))
 (arc (start 91.954 27.793499) (mid 90.768 26.6075) (end 89.582 27.793499) (width 2.115) (layer "F.Cu") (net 2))
 (arc (start 49.257999 36.313357) (mid 48.071999 35.127357) (end 46.885999 36.313357) (width 2.115) (layer "F.Cu") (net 2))
 (arc (start 47.793499 101.442) (mid 46.607499 102.628) (end 47.793499 103.814) (width 2.115) (layer "F.Cu") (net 2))
 (arc (start 96.698 34.043499) (mid 95.512 32.857499) (end 94.326 34.043499) (width 2.115) (layer "F.Cu") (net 2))
 (arc (start 82.466 27.793499) (mid 81.279999 26.6075) (end 80.094 27.793499) (width 2.115) (layer "F.Cu") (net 2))
 (arc (start 68.234 27.793499) (mid 67.048 26.6075) (end 65.862 27.793499) (width 2.115) (layer "F.Cu") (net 2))
 (arc (start 102.384499 94.326) (mid 103.5705 95.512) (end 102.384499 96.698) (width 2.115) (layer "F.Cu") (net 2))
 (arc (start 61.118 86.023999) (mid 59.932 87.21) (end 58.746 86.023999) (width 2.115) (layer "F.Cu") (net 2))
 (arc (start 65.862 86.023999) (mid 64.676 87.21) (end 63.489999 86.023999) (width 2.115) (layer "F.Cu") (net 2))
 (arc (start 47.793499 91.954) (mid 46.607499 93.14) (end 47.793499 94.326) (width 2.115) (layer "F.Cu") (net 2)))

